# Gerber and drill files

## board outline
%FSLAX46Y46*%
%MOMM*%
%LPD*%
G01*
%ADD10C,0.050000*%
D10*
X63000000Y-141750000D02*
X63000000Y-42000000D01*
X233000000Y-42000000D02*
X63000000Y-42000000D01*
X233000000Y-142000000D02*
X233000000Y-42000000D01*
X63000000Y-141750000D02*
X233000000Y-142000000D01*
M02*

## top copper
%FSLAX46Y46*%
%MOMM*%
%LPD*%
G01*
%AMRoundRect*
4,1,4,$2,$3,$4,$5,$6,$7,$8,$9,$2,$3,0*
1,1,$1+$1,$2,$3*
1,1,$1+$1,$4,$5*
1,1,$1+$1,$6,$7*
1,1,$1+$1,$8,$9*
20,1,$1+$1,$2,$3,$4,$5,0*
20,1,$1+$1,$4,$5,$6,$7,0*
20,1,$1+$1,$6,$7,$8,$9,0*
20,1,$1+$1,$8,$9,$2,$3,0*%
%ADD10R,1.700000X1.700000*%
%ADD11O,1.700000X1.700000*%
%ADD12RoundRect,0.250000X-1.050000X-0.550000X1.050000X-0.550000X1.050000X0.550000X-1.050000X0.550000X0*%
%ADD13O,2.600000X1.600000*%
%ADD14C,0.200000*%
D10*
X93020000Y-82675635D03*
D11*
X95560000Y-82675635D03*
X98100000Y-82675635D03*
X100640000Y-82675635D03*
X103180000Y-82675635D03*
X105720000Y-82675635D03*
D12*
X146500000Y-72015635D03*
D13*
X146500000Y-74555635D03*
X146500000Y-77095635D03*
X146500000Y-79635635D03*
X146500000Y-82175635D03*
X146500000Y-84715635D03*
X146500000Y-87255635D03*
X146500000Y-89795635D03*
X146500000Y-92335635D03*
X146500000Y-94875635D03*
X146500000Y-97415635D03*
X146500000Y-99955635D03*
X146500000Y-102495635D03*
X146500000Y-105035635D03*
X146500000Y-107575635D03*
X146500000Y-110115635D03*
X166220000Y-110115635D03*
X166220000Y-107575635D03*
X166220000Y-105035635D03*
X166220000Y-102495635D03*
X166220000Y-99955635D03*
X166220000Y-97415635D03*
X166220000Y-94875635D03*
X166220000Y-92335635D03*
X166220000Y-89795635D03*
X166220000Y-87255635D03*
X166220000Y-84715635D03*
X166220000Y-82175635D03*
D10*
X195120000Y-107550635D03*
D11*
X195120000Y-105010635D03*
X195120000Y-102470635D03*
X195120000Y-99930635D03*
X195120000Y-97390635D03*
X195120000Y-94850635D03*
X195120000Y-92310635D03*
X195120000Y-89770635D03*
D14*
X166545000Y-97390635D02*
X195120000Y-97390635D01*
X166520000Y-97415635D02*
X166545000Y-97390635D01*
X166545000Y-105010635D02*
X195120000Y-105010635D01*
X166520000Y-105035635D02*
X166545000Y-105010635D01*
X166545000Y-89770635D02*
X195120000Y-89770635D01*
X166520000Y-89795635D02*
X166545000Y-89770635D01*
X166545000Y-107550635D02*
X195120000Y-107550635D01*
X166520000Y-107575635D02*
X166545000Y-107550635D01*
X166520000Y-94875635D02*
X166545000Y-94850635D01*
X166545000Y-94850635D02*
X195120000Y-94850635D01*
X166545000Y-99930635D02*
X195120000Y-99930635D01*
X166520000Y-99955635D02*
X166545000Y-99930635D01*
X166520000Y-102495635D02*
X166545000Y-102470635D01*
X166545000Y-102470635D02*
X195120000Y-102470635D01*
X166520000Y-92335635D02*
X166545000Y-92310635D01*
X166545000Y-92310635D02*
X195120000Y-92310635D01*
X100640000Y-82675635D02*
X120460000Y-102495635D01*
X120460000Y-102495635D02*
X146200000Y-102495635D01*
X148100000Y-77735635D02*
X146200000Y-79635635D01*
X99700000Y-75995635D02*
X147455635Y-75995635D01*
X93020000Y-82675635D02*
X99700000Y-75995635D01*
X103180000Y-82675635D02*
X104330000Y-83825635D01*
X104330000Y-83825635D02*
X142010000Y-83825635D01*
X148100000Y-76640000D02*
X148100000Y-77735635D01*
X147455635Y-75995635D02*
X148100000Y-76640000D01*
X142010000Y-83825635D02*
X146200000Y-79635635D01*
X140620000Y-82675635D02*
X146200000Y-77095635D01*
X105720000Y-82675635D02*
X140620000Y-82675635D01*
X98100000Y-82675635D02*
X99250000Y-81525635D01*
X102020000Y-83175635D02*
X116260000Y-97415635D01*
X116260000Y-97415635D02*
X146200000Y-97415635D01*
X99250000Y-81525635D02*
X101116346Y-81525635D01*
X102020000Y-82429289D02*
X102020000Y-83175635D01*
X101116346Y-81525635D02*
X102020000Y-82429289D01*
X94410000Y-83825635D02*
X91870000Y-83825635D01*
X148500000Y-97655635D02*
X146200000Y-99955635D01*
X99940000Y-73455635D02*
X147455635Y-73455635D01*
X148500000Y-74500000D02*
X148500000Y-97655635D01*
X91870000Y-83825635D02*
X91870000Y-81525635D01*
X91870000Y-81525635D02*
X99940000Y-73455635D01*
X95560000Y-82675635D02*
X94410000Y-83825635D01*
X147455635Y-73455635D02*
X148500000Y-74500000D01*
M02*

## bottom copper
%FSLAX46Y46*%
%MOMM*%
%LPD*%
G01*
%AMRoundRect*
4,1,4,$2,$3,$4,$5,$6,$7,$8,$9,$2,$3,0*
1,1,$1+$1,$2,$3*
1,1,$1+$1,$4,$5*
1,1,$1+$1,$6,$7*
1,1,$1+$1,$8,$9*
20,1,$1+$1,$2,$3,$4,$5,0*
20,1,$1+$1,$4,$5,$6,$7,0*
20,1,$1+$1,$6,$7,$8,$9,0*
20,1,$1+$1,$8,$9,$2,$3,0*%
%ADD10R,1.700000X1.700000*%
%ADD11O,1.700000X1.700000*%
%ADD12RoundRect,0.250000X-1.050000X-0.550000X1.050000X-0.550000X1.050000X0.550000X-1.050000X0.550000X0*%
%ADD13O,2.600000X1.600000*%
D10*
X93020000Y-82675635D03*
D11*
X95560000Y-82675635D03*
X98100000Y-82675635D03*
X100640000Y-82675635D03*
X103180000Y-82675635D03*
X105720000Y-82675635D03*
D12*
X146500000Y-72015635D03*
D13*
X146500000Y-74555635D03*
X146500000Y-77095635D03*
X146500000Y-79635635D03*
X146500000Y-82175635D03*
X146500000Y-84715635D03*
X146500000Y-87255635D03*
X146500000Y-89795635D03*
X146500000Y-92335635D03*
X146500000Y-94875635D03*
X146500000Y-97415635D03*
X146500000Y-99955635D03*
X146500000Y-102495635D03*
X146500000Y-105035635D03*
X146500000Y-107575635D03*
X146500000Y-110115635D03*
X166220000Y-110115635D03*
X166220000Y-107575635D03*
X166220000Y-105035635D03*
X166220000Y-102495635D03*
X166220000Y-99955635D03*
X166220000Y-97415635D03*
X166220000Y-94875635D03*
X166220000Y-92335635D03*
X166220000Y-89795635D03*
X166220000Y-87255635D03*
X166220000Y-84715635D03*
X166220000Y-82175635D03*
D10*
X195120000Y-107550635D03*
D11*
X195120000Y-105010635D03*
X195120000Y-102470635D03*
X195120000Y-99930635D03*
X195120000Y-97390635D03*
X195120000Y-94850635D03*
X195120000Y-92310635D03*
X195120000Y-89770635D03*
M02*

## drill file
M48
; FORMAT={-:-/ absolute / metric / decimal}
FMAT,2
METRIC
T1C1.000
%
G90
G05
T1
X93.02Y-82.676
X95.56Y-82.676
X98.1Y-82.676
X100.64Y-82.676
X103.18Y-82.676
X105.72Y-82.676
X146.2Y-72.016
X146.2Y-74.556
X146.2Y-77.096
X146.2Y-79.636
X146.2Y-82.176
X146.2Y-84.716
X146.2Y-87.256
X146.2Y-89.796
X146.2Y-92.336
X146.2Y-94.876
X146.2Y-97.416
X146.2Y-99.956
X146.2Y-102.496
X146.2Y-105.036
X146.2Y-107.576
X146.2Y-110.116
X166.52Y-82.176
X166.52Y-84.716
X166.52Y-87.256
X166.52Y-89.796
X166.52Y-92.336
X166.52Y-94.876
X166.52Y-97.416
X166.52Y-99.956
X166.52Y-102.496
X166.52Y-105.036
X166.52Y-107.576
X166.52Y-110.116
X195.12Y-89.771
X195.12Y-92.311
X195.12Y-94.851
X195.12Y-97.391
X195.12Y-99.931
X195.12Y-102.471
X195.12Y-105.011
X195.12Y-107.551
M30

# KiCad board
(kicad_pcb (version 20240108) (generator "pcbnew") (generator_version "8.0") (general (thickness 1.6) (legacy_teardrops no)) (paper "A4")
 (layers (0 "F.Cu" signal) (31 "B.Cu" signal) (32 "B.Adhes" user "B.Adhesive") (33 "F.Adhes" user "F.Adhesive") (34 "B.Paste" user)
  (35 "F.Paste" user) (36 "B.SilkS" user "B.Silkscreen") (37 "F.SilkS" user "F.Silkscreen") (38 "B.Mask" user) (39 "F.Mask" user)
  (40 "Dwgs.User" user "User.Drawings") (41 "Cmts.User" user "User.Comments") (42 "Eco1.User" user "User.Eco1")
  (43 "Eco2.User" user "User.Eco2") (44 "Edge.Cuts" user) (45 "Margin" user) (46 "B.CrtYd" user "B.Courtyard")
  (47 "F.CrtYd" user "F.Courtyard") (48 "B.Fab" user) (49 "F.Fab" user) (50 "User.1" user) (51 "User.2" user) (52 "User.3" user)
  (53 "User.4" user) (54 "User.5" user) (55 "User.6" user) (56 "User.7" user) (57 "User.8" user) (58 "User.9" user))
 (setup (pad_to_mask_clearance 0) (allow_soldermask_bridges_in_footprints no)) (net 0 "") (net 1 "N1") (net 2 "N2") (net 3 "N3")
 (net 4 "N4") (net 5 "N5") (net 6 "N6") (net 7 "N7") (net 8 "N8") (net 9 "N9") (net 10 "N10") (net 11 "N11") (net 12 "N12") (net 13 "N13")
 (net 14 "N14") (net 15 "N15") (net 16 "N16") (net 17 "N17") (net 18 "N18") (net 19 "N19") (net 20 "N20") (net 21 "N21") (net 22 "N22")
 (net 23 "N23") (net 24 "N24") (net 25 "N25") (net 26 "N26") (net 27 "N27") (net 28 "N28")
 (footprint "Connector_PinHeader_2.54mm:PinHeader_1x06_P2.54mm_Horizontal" (layer "F.Cu") (at 93.02 82.675635 90)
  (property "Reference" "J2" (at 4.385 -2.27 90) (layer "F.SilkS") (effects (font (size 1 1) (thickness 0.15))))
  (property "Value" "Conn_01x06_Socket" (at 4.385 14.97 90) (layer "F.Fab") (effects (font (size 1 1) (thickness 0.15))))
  (pad "1" thru_hole rect (at 0 0 90) (size 1.7 1.7) (drill 1) (layers "*.Cu" "*.Mask") (remove_unused_layers no) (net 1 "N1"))
  (pad "2" thru_hole oval (at 0 2.54 90) (size 1.7 1.7) (drill 1) (layers "*.Cu" "*.Mask") (remove_unused_layers no) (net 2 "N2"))
  (pad "3" thru_hole oval (at 0 5.08 90) (size 1.7 1.7) (drill 1) (layers "*.Cu" "*.Mask") (remove_unused_layers no) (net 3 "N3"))
  (pad "4" thru_hole oval (at 0 7.62 90) (size 1.7 1.7) (drill 1) (layers "*.Cu" "*.Mask") (remove_unused_layers no) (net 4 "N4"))
  (pad "5" thru_hole oval (at 0 10.16 90) (size 1.7 1.7) (drill 1) (layers "*.Cu" "*.Mask") (remove_unused_layers no) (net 1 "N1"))
  (pad "6" thru_hole oval (at 0 12.7 90) (size 1.7 1.7) (drill 1) (layers "*.Cu" "*.Mask") (remove_unused_layers no) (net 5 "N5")))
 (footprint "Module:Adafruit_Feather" (layer "F.Cu") (at 146.2 72.015635)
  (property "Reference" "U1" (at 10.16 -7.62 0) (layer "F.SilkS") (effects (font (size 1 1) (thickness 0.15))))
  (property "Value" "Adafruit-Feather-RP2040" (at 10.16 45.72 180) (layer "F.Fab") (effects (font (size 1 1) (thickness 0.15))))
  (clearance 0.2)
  (pad "1" thru_hole roundrect (at 0 0) (size 2.6 1.6) (drill 1 (offset 0.3 0)) (layers "*.Cu" "*.Mask") (remove_unused_layers no)
   (roundrect_rratio 0.15625) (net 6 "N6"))
  (pad "2" thru_hole oval (at 0 2.54) (size 2.6 1.6) (drill 1 (offset 0.3 0)) (layers "*.Cu" "*.Mask") (remove_unused_layers no)
   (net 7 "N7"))
  (pad "3" thru_hole oval (at 0 5.08) (size 2.6 1.6) (drill 1 (offset 0.3 0)) (layers "*.Cu" "*.Mask") (remove_unused_layers no)
   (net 5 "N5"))
  (pad "4" thru_hole oval (at 0 7.62) (size 2.6 1.6) (drill 1 (offset 0.3 0)) (layers "*.Cu" "*.Mask") (remove_unused_layers no)
   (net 1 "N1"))
  (pad "5" thru_hole oval (at 0 10.16) (size 2.6 1.6) (drill 1 (offset 0.3 0)) (layers "*.Cu" "*.Mask") (remove_unused_layers no)
   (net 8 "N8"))
  (pad "6" thru_hole oval (at 0 12.7) (size 2.6 1.6) (drill 1 (offset 0.3 0)) (layers "*.Cu" "*.Mask") (remove_unused_layers no)
   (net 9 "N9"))
  (pad "7" thru_hole oval (at 0 15.24) (size 2.6 1.6) (drill 1 (offset 0.3 0)) (layers "*.Cu" "*.Mask") (remove_unused_layers no)
   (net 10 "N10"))
  (pad "8" thru_hole oval (at 0 17.78) (size 2.6 1.6) (drill 1 (offset 0.3 0)) (layers "*.Cu" "*.Mask") (remove_unused_layers no)
   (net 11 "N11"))
  (pad "9" thru_hole oval (at 0 20.32) (size 2.6 1.6) (drill 1 (offset 0.3 0)) (layers "*.Cu" "*.Mask") (remove_unused_layers no)
   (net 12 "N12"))
  (pad "10" thru_hole oval (at 0 22.86) (size 2.6 1.6) (drill 1 (offset 0.3 0)) (layers "*.Cu" "*.Mask") (remove_unused_layers no)
   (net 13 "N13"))
  (pad "11" thru_hole oval (at 0 25.4) (size 2.6 1.6) (drill 1 (offset 0.3 0)) (layers "*.Cu" "*.Mask") (remove_unused_layers no)
   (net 3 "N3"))
  (pad "12" thru_hole oval (at 0 27.94) (size 2.6 1.6) (drill 1 (offset 0.3 0)) (layers "*.Cu" "*.Mask") (remove_unused_layers no)
   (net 2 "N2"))
  (pad "13" thru_hole oval (at 0 30.48) (size 2.6 1.6) (drill 1 (offset 0.3 0)) (layers "*.Cu" "*.Mask") (remove_unused_layers no)
   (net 4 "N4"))
  (pad "14" thru_hole oval (at 0 33.02) (size 2.6 1.6) (drill 1 (offset 0.3 0)) (layers "*.Cu" "*.Mask") (remove_unused_layers no)
   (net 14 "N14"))
  (pad "15" thru_hole oval (at 0 35.56) (size 2.6 1.6) (drill 1 (offset 0.3 0)) (layers "*.Cu" "*.Mask") (remove_unused_layers no)
   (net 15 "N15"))
  (pad "16" thru_hole oval (at 0 38.1) (size 2.6 1.6) (drill 1 (offset 0.3 0)) (layers "*.Cu" "*.Mask") (remove_unused_layers no)
   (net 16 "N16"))
  (pad "17" thru_hole oval (at 20.32 38.1 180) (size 2.6 1.6) (drill 1 (offset 0.3 0)) (layers "*.Cu" "*.Mask") (remove_unused_layers no)
   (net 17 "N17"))
  (pad "18" thru_hole oval (at 20.32 35.56 180) (size 2.6 1.6) (drill 1 (offset 0.3 0)) (layers "*.Cu" "*.Mask") (remove_unused_layers no)
   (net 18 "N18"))
  (pad "19" thru_hole oval (at 20.32 33.02 180) (size 2.6 1.6) (drill 1 (offset 0.3 0)) (layers "*.Cu" "*.Mask") (remove_unused_layers no)
   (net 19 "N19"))
  (pad "20" thru_hole oval (at 20.32 30.48 180) (size 2.6 1.6) (drill 1 (offset 0.3 0)) (layers "*.Cu" "*.Mask") (remove_unused_layers no)
   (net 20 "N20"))
  (pad "21" thru_hole oval (at 20.32 27.94 180) (size 2.6 1.6) (drill 1 (offset 0.3 0)) (layers "*.Cu" "*.Mask") (remove_unused_layers no)
   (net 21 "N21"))
  (pad "22" thru_hole oval (at 20.32 25.4 180) (size 2.6 1.6) (drill 1 (offset 0.3 0)) (layers "*.Cu" "*.Mask") (remove_unused_layers no)
   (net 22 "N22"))
  (pad "23" thru_hole oval (at 20.32 22.86 180) (size 2.6 1.6) (drill 1 (offset 0.3 0)) (layers "*.Cu" "*.Mask") (remove_unused_layers no)
   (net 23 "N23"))
  (pad "24" thru_hole oval (at 20.32 20.32 180) (size 2.6 1.6) (drill 1 (offset 0.3 0)) (layers "*.Cu" "*.Mask") (remove_unused_layers no)
   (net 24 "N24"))
  (pad "25" thru_hole oval (at 20.32 17.78 180) (size 2.6 1.6) (drill 1 (offset 0.3 0)) (layers "*.Cu" "*.Mask") (remove_unused_layers no)
   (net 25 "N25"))
  (pad "26" thru_hole oval (at 20.32 15.24 180) (size 2.6 1.6) (drill 1 (offset 0.3 0)) (layers "*.Cu" "*.Mask") (remove_unused_layers no)
   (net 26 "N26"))
  (pad "27" thru_hole oval (at 20.32 12.7 180) (size 2.6 1.6) (drill 1 (offset 0.3 0)) (layers "*.Cu" "*.Mask") (remove_unused_layers no)
   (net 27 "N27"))
  (pad "28" thru_hole oval (at 20.32 10.16 180) (size 2.6 1.6) (drill 1 (offset 0.3 0)) (layers "*.Cu" "*.Mask") (remove_unused_layers no)
   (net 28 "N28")))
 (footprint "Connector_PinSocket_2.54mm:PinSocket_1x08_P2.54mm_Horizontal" (layer "F.Cu") (at 195.12 107.550635 180)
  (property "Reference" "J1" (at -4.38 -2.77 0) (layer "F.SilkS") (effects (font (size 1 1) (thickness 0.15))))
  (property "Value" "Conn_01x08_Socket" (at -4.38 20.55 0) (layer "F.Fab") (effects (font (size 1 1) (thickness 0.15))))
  (pad "1" thru_hole rect (at 0 0 180) (size 1.7 1.7) (drill 1) (layers "*.Cu" "*.Mask") (remove_unused_layers no) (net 18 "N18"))
  (pad "2" thru_hole oval (at 0 2.54 180) (size 1.7 1.7) (drill 1) (layers "*.Cu" "*.Mask") (remove_unused_layers no) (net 19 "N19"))
  (pad "3" thru_hole oval (at 0 5.08 180) (size 1.7 1.7) (drill 1) (layers "*.Cu" "*.Mask") (remove_unused_layers no) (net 20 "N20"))
  (pad "4" thru_hole oval (at 0 7.62 180) (size 1.7 1.7) (drill 1) (layers "*.Cu" "*.Mask") (remove_unused_layers no) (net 21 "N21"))
  (pad "5" thru_hole oval (at 0 10.16 180) (size 1.7 1.7) (drill 1) (layers "*.Cu" "*.Mask") (remove_unused_layers no) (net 22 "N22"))
  (pad "6" thru_hole oval (at 0 12.7 180) (size 1.7 1.7) (drill 1) (layers "*.Cu" "*.Mask") (remove_unused_layers no) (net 23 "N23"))
  (pad "7" thru_hole oval (at 0 15.24 180) (size 1.7 1.7) (drill 1) (layers "*.Cu" "*.Mask") (remove_unused_layers no) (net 24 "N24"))
  (pad "8" thru_hole oval (at 0 17.78 180) (size 1.7 1.7) (drill 1) (layers "*.Cu" "*.Mask") (remove_unused_layers no) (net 25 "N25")))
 (gr_line (start 63 141.75) (end 63 42) (stroke (width 0.05) (type default)) (layer "Edge.Cuts"))
 (gr_line (start 233 42) (end 63 42) (stroke (width 0.05) (type default)) (layer "Edge.Cuts"))
 (gr_line (start 233 142) (end 233 42) (stroke (width 0.05) (type default)) (layer "Edge.Cuts"))
 (gr_line (start 63 141.75) (end 233 142) (stroke (width 0.05) (type default)) (layer "Edge.Cuts"))
 (segment (start 166.545 97.390635) (end 195.12 97.390635) (width 0.2) (layer "F.Cu") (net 22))
 (segment (start 166.52 97.415635) (end 166.545 97.390635) (width 0.2) (layer "F.Cu") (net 22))
 (segment (start 166.545 105.010635) (end 195.12 105.010635) (width 0.2) (layer "F.Cu") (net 19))
 (segment (start 166.52 105.035635) (end 166.545 105.010635) (width 0.2) (layer "F.Cu") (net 19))
 (segment (start 166.545 89.770635) (end 195.12 89.770635) (width 0.2) (layer "F.Cu") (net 25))
 (segment (start 166.52 89.795635) (end 166.545 89.770635) (width 0.2) (layer "F.Cu") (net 25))
 (segment (start 166.545 107.550635) (end 195.12 107.550635) (width 0.2) (layer "F.Cu") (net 18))
 (segment (start 166.52 107.575635) (end 166.545 107.550635) (width 0.2) (layer "F.Cu") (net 18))
 (segment (start 166.52 94.875635) (end 166.545 94.850635) (width 0.2) (layer "F.Cu") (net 23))
 (segment (start 166.545 94.850635) (end 195.12 94.850635) (width 0.2) (layer "F.Cu") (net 23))
 (segment (start 166.545 99.930635) (end 195.12 99.930635) (width 0.2) (layer "F.Cu") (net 21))
 (segment (start 166.52 99.955635) (end 166.545 99.930635) (width 0.2) (layer "F.Cu") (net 21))
 (segment (start 166.52 102.495635) (end 166.545 102.470635) (width 0.2) (layer "F.Cu") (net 20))
 (segment (start 166.545 102.470635) (end 195.12 102.470635) (width 0.2) (layer "F.Cu") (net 20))
 (segment (start 166.52 92.335635) (end 166.545 92.310635) (width 0.2) (layer "F.Cu") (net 24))
 (segment (start 166.545 92.310635) (end 195.12 92.310635) (width 0.2) (layer "F.Cu") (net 24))
 (segment (start 100.64 82.675635) (end 120.46 102.495635) (width 0.2) (layer "F.Cu") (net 4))
 (segment (start 120.46 102.495635) (end 146.2 102.495635) (width 0.2) (layer "F.Cu") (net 4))
 (segment (start 148.1 77.735635) (end 146.2 79.635635) (width 0.2) (layer "F.Cu") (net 1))
 (segment (start 99.7 75.995635) (end 147.455635 75.995635) (width 0.2) (layer "F.Cu") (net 1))
 (segment (start 93.02 82.675635) (end 99.7 75.995635) (width 0.2) (layer "F.Cu") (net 1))
 (segment (start 103.18 82.675635) (end 104.33 83.825635) (width 0.2) (layer "F.Cu") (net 1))
 (segment (start 104.33 83.825635) (end 142.01 83.825635) (width 0.2) (layer "F.Cu") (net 1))
 (segment (start 148.1 76.64) (end 148.1 77.735635) (width 0.2) (layer "F.Cu") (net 1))
 (segment (start 147.455635 75.995635) (end 148.1 76.64) (width 0.2) (layer "F.Cu") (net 1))
 (segment (start 142.01 83.825635) (end 146.2 79.635635) (width 0.2) (layer "F.Cu") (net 1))
 (segment (start 140.62 82.675635) (end 146.2 77.095635) (width 0.2) (layer "F.Cu") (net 5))
 (segment (start 105.72 82.675635) (end 140.62 82.675635) (width 0.2) (layer "F.Cu") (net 5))
 (segment (start 98.1 82.675635) (end 99.25 81.525635) (width 0.2) (layer "F.Cu") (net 3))
 (segment (start 102.02 83.175635) (end 116.26 97.415635) (width 0.2) (layer "F.Cu") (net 3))
 (segment (start 116.26 97.415635) (end 146.2 97.415635) (width 0.2) (layer "F.Cu") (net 3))
 (segment (start 99.25 81.525635) (end 101.116346 81.525635) (width 0.2) (layer "F.Cu") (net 3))
 (segment (start 102.02 82.429289) (end 102.02 83.175635) (width 0.2) (layer "F.Cu") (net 3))
 (segment (start 101.116346 81.525635) (end 102.02 82.429289) (width 0.2) (layer "F.Cu") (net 3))
 (segment (start 94.41 83.825635) (end 91.87 83.825635) (width 0.2) (layer "F.Cu") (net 2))
 (segment (start 148.5 97.655635) (end 146.2 99.955635) (width 0.2) (layer "F.Cu") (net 2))
 (segment (start 99.94 73.455635) (end 147.455635 73.455635) (width 0.2) (layer "F.Cu") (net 2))
 (segment (start 148.5 74.5) (end 148.5 97.655635) (width 0.2) (layer "F.Cu") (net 2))
 (segment (start 91.87 83.825635) (end 91.87 81.525635) (width 0.2) (layer "F.Cu") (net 2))
 (segment (start 91.87 81.525635) (end 99.94 73.455635) (width 0.2) (layer "F.Cu") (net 2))
 (segment (start 95.56 82.675635) (end 94.41 83.825635) (width 0.2) (layer "F.Cu") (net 2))
 (segment (start 147.455635 73.455635) (end 148.5 74.5) (width 0.2) (layer "F.Cu") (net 2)))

